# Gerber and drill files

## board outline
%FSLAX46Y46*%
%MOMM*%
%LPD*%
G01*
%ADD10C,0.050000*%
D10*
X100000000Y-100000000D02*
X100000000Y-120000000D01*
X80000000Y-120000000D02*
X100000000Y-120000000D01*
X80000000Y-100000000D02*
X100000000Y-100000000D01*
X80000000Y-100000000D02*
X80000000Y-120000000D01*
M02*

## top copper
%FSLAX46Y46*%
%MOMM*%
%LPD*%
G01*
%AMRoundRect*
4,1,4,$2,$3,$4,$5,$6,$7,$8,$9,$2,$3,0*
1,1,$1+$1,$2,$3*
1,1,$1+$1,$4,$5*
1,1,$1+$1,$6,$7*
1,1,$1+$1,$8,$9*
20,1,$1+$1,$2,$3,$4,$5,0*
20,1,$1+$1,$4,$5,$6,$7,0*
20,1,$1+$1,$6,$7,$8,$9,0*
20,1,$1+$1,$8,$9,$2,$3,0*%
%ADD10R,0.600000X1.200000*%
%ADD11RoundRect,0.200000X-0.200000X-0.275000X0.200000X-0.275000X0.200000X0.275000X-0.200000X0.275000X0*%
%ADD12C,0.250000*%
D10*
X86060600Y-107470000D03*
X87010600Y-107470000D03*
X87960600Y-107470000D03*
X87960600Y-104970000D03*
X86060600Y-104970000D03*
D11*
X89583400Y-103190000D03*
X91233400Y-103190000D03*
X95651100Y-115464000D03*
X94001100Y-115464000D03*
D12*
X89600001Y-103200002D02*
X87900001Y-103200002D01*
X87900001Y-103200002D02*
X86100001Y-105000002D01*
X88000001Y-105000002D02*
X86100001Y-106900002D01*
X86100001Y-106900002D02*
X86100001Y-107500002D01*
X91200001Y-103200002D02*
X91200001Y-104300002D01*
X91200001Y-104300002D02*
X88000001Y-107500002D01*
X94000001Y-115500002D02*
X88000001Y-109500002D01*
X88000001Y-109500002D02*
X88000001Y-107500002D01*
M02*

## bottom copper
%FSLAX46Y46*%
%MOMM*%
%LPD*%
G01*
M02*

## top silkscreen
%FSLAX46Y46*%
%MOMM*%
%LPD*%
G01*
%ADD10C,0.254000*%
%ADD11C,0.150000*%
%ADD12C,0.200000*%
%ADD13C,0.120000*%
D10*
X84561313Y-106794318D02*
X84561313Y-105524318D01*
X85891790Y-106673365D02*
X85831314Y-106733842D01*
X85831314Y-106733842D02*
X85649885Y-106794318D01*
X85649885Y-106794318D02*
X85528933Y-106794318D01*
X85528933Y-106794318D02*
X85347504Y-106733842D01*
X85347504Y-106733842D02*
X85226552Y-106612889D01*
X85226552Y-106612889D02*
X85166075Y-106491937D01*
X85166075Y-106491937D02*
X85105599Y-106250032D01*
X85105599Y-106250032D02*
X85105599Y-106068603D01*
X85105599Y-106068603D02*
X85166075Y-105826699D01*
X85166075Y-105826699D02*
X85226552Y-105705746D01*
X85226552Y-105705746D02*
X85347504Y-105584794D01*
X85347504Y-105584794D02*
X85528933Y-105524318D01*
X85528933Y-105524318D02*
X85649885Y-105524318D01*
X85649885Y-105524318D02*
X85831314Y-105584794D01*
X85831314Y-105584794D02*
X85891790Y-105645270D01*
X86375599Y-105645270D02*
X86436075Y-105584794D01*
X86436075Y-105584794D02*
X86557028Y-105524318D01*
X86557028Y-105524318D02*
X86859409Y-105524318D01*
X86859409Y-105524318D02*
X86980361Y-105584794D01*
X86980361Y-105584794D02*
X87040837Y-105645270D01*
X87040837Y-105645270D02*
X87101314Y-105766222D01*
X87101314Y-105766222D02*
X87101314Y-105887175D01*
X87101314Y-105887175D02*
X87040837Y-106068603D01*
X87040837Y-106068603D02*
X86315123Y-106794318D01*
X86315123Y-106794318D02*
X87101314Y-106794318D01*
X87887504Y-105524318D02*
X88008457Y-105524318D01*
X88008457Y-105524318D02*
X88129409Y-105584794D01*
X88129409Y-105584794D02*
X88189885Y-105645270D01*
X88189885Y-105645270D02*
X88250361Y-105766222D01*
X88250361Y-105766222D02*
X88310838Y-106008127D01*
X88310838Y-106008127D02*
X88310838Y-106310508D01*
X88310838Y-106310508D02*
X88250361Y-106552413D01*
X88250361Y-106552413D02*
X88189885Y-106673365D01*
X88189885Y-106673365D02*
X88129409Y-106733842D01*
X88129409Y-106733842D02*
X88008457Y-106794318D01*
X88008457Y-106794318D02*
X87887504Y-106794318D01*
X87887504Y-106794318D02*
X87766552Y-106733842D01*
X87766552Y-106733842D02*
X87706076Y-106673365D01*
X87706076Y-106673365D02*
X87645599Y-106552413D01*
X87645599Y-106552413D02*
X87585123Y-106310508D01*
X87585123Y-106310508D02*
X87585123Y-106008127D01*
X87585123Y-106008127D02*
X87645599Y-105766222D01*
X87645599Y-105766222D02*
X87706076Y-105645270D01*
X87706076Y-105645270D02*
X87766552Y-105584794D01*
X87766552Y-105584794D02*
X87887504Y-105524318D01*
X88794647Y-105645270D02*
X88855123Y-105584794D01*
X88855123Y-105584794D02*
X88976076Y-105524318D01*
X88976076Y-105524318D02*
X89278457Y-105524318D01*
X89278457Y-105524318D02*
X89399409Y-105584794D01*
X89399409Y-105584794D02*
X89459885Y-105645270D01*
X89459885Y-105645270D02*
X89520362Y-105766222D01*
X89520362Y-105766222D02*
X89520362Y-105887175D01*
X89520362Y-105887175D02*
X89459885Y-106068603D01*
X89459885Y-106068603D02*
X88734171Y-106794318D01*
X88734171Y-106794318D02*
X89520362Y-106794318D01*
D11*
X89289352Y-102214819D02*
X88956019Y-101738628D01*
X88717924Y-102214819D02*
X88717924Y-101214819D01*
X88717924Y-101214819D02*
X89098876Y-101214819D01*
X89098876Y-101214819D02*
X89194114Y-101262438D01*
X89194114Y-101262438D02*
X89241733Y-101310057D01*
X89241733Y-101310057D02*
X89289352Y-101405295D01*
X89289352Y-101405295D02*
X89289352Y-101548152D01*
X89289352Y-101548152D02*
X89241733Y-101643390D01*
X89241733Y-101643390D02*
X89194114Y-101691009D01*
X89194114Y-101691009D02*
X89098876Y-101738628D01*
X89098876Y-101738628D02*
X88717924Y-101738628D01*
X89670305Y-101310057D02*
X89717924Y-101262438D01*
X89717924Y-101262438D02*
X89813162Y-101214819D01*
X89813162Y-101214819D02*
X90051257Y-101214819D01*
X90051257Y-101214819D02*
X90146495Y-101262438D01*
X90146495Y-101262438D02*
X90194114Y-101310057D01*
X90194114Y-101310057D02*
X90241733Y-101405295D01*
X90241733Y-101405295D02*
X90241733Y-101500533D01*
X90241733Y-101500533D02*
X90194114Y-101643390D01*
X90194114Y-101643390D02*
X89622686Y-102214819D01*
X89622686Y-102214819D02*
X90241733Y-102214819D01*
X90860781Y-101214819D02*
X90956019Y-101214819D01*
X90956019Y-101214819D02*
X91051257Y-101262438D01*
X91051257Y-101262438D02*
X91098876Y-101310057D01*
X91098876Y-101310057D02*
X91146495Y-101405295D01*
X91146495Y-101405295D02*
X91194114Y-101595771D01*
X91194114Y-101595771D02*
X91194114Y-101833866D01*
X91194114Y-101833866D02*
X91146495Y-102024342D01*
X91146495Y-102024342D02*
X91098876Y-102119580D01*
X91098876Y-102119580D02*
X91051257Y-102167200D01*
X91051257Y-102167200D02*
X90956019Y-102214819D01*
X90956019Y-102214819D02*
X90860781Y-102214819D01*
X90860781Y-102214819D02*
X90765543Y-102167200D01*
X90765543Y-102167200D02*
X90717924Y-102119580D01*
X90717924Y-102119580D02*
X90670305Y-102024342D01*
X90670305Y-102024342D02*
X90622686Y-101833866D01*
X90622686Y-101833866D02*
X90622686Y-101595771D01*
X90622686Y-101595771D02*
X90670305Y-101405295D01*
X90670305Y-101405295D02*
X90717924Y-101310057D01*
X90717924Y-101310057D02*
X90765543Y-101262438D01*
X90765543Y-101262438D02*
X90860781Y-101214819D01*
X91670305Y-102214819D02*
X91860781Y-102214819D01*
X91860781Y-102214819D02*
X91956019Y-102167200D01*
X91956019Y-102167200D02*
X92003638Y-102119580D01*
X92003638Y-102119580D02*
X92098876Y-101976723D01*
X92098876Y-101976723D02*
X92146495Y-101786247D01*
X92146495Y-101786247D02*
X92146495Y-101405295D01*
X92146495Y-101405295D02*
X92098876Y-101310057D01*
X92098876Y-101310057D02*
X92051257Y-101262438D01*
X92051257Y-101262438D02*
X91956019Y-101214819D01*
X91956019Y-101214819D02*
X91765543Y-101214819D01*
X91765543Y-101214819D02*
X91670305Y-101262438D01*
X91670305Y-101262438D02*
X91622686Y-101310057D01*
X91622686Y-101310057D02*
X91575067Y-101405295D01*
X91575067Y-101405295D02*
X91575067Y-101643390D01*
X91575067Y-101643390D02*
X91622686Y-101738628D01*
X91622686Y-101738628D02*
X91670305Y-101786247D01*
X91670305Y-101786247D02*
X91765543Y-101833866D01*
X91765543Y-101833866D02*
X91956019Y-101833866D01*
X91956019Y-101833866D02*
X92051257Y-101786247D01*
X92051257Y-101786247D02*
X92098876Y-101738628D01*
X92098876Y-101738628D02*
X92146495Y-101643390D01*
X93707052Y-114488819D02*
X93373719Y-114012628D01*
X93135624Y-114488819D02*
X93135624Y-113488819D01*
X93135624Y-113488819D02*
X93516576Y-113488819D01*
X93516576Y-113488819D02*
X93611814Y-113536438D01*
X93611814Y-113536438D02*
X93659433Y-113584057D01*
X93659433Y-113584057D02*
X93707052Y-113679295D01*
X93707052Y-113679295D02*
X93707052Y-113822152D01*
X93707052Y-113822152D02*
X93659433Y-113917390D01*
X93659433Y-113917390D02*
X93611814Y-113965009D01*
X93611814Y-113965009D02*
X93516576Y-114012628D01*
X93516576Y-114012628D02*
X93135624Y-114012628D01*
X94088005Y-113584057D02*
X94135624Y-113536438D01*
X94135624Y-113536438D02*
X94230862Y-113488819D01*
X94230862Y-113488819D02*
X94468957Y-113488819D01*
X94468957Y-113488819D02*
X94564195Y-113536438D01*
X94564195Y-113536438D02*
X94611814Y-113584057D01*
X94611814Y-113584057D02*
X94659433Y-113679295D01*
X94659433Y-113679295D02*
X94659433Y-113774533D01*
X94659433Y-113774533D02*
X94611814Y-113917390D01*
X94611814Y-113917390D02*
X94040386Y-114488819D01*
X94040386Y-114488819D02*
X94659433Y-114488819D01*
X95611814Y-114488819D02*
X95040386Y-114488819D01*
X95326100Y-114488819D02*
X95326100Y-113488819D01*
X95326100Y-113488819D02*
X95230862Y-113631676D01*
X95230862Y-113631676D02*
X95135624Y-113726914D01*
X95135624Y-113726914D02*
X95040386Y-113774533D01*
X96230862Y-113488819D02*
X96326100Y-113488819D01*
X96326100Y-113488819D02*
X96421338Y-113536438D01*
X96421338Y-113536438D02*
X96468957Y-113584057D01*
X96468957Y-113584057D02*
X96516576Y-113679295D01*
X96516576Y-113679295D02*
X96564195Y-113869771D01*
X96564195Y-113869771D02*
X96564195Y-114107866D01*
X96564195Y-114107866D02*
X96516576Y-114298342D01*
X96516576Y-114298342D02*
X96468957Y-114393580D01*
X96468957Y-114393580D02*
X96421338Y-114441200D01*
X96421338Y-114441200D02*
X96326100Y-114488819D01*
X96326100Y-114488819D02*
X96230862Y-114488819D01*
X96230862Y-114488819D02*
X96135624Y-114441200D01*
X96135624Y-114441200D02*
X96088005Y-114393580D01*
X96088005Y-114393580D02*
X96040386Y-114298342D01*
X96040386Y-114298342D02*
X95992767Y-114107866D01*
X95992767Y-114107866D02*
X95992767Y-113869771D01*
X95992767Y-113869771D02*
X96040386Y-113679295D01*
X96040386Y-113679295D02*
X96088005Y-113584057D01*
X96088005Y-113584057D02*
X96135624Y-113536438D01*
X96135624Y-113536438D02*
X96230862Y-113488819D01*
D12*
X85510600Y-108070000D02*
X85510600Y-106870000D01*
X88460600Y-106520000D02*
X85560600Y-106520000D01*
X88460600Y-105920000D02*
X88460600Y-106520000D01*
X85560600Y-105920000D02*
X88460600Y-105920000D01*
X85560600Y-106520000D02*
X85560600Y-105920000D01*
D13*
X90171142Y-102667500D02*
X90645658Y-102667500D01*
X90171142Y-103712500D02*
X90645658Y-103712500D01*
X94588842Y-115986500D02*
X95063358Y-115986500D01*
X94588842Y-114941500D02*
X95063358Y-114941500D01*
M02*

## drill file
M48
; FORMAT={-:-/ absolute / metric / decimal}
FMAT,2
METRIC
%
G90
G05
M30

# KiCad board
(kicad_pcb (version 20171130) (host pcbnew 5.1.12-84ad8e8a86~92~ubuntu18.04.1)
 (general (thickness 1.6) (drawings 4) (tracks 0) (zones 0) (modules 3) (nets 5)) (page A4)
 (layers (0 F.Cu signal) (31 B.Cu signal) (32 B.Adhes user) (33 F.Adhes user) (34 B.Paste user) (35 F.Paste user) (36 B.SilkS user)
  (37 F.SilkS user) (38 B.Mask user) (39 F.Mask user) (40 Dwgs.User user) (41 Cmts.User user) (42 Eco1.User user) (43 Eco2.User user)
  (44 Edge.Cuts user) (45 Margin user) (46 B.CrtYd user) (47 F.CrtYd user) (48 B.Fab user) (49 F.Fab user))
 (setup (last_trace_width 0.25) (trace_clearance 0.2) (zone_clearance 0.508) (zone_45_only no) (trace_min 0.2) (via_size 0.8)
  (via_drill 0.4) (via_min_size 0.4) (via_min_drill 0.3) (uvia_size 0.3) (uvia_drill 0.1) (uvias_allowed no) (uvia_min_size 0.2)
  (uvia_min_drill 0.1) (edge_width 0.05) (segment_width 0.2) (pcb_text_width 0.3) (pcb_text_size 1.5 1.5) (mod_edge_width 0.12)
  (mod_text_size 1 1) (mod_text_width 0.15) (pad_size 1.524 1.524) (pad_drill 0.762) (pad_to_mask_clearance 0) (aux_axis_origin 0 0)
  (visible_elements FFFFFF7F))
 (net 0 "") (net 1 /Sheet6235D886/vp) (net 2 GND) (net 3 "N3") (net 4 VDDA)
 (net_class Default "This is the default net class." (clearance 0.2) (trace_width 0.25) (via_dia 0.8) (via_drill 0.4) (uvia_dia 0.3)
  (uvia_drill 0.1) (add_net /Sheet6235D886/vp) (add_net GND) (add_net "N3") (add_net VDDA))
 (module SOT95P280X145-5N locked (layer F.Cu) (at 87.010600 106.220000 90.000000)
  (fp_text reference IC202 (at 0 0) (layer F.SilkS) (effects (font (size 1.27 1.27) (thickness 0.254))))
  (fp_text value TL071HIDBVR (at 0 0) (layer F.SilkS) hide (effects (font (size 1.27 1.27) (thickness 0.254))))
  (fp_line (start -1.85 -1.5) (end -0.65 -1.5) (layer F.SilkS) (width 0.2))
  (fp_line (start -0.3 1.45) (end -0.3 -1.45) (layer F.SilkS) (width 0.2))
  (fp_line (start 0.3 1.45) (end -0.3 1.45) (layer F.SilkS) (width 0.2))
  (fp_line (start 0.3 -1.45) (end 0.3 1.45) (layer F.SilkS) (width 0.2))
  (fp_line (start -0.3 -1.45) (end 0.3 -1.45) (layer F.SilkS) (width 0.2))
  (pad 1 smd rect (at -1.25 -0.95 180.000000) (size 0.6 1.2) (layers F.Cu F.Mask F.Paste) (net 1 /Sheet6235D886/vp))
  (pad 2 smd rect (at -1.25 0 180.000000) (size 0.6 1.2) (layers F.Cu F.Mask F.Paste) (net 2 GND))
  (pad 3 smd rect (at -1.25 0.95 180.000000) (size 0.6 1.2) (layers F.Cu F.Mask F.Paste) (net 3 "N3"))
  (pad 4 smd rect (at 1.25 0.95 180.000000) (size 0.6 1.2) (layers F.Cu F.Mask F.Paste) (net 1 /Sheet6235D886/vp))
  (pad 5 smd rect (at 1.25 -0.95 180.000000) (size 0.6 1.2) (layers F.Cu F.Mask F.Paste) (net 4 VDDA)))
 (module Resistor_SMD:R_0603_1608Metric (layer F.Cu) (at 90.408400 103.190000)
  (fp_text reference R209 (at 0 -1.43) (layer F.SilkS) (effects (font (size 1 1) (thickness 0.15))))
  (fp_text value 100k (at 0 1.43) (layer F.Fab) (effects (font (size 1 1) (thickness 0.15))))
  (fp_line (start -0.237258 -0.5225) (end 0.237258 -0.5225) (layer F.SilkS) (width 0.12))
  (fp_line (start -0.237258 0.5225) (end 0.237258 0.5225) (layer F.SilkS) (width 0.12))
  (pad 1 smd roundrect (at -0.825 0) (size 0.8 0.95) (layers F.Cu F.Mask F.Paste) (roundrect_rratio 0.25) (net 4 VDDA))
  (pad 2 smd roundrect (at 0.825 0) (size 0.8 0.95) (layers F.Cu F.Mask F.Paste) (roundrect_rratio 0.25) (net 3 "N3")))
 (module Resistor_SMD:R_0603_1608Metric (layer F.Cu) (at 94.826100 115.464000)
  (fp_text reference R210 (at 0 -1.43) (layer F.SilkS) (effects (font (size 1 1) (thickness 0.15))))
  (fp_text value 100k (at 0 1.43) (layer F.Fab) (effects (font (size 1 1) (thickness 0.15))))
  (fp_line (start -0.237258 0.5225) (end 0.237258 0.5225) (layer F.SilkS) (width 0.12))
  (fp_line (start -0.237258 -0.5225) (end 0.237258 -0.5225) (layer F.SilkS) (width 0.12))
  (pad 2 smd roundrect (at 0.825 0) (size 0.8 0.95) (layers F.Cu F.Mask F.Paste) (roundrect_rratio 0.25) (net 2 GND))
  (pad 1 smd roundrect (at -0.825 0) (size 0.8 0.95) (layers F.Cu F.Mask F.Paste) (roundrect_rratio 0.25) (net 3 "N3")))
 (gr_line (start 100 100) (end 100 120) (layer Edge.Cuts) (width 0.05))
 (gr_line (start 80 120) (end 100 120) (layer Edge.Cuts) (width 0.05))
 (gr_line (start 80 100) (end 100 100) (layer Edge.Cuts) (width 0.05))
 (gr_line (start 80 100) (end 80 120) (layer Edge.Cuts) (width 0.05))
 (segment (start 89.600001 103.200002) (end 87.900001 103.200002) (width 0.250000) (layer F.Cu) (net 4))
 (segment (start 87.900001 103.200002) (end 86.100001 105.000002) (width 0.250000) (layer F.Cu) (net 4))
 (segment (start 88.000001 105.000002) (end 86.100001 106.900002) (width 0.250000) (layer F.Cu) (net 1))
 (segment (start 86.100001 106.900002) (end 86.100001 107.500002) (width 0.250000) (layer F.Cu) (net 1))
 (segment (start 91.200001 103.200002) (end 91.200001 104.300002) (width 0.250000) (layer F.Cu) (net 3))
 (segment (start 91.200001 104.300002) (end 88.000001 107.500002) (width 0.250000) (layer F.Cu) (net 3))
 (segment (start 94.000001 115.500002) (end 88.000001 109.500002) (width 0.250000) (layer F.Cu) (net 3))
 (segment (start 88.000001 109.500002) (end 88.000001 107.500002) (width 0.250000) (layer F.Cu) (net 3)))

